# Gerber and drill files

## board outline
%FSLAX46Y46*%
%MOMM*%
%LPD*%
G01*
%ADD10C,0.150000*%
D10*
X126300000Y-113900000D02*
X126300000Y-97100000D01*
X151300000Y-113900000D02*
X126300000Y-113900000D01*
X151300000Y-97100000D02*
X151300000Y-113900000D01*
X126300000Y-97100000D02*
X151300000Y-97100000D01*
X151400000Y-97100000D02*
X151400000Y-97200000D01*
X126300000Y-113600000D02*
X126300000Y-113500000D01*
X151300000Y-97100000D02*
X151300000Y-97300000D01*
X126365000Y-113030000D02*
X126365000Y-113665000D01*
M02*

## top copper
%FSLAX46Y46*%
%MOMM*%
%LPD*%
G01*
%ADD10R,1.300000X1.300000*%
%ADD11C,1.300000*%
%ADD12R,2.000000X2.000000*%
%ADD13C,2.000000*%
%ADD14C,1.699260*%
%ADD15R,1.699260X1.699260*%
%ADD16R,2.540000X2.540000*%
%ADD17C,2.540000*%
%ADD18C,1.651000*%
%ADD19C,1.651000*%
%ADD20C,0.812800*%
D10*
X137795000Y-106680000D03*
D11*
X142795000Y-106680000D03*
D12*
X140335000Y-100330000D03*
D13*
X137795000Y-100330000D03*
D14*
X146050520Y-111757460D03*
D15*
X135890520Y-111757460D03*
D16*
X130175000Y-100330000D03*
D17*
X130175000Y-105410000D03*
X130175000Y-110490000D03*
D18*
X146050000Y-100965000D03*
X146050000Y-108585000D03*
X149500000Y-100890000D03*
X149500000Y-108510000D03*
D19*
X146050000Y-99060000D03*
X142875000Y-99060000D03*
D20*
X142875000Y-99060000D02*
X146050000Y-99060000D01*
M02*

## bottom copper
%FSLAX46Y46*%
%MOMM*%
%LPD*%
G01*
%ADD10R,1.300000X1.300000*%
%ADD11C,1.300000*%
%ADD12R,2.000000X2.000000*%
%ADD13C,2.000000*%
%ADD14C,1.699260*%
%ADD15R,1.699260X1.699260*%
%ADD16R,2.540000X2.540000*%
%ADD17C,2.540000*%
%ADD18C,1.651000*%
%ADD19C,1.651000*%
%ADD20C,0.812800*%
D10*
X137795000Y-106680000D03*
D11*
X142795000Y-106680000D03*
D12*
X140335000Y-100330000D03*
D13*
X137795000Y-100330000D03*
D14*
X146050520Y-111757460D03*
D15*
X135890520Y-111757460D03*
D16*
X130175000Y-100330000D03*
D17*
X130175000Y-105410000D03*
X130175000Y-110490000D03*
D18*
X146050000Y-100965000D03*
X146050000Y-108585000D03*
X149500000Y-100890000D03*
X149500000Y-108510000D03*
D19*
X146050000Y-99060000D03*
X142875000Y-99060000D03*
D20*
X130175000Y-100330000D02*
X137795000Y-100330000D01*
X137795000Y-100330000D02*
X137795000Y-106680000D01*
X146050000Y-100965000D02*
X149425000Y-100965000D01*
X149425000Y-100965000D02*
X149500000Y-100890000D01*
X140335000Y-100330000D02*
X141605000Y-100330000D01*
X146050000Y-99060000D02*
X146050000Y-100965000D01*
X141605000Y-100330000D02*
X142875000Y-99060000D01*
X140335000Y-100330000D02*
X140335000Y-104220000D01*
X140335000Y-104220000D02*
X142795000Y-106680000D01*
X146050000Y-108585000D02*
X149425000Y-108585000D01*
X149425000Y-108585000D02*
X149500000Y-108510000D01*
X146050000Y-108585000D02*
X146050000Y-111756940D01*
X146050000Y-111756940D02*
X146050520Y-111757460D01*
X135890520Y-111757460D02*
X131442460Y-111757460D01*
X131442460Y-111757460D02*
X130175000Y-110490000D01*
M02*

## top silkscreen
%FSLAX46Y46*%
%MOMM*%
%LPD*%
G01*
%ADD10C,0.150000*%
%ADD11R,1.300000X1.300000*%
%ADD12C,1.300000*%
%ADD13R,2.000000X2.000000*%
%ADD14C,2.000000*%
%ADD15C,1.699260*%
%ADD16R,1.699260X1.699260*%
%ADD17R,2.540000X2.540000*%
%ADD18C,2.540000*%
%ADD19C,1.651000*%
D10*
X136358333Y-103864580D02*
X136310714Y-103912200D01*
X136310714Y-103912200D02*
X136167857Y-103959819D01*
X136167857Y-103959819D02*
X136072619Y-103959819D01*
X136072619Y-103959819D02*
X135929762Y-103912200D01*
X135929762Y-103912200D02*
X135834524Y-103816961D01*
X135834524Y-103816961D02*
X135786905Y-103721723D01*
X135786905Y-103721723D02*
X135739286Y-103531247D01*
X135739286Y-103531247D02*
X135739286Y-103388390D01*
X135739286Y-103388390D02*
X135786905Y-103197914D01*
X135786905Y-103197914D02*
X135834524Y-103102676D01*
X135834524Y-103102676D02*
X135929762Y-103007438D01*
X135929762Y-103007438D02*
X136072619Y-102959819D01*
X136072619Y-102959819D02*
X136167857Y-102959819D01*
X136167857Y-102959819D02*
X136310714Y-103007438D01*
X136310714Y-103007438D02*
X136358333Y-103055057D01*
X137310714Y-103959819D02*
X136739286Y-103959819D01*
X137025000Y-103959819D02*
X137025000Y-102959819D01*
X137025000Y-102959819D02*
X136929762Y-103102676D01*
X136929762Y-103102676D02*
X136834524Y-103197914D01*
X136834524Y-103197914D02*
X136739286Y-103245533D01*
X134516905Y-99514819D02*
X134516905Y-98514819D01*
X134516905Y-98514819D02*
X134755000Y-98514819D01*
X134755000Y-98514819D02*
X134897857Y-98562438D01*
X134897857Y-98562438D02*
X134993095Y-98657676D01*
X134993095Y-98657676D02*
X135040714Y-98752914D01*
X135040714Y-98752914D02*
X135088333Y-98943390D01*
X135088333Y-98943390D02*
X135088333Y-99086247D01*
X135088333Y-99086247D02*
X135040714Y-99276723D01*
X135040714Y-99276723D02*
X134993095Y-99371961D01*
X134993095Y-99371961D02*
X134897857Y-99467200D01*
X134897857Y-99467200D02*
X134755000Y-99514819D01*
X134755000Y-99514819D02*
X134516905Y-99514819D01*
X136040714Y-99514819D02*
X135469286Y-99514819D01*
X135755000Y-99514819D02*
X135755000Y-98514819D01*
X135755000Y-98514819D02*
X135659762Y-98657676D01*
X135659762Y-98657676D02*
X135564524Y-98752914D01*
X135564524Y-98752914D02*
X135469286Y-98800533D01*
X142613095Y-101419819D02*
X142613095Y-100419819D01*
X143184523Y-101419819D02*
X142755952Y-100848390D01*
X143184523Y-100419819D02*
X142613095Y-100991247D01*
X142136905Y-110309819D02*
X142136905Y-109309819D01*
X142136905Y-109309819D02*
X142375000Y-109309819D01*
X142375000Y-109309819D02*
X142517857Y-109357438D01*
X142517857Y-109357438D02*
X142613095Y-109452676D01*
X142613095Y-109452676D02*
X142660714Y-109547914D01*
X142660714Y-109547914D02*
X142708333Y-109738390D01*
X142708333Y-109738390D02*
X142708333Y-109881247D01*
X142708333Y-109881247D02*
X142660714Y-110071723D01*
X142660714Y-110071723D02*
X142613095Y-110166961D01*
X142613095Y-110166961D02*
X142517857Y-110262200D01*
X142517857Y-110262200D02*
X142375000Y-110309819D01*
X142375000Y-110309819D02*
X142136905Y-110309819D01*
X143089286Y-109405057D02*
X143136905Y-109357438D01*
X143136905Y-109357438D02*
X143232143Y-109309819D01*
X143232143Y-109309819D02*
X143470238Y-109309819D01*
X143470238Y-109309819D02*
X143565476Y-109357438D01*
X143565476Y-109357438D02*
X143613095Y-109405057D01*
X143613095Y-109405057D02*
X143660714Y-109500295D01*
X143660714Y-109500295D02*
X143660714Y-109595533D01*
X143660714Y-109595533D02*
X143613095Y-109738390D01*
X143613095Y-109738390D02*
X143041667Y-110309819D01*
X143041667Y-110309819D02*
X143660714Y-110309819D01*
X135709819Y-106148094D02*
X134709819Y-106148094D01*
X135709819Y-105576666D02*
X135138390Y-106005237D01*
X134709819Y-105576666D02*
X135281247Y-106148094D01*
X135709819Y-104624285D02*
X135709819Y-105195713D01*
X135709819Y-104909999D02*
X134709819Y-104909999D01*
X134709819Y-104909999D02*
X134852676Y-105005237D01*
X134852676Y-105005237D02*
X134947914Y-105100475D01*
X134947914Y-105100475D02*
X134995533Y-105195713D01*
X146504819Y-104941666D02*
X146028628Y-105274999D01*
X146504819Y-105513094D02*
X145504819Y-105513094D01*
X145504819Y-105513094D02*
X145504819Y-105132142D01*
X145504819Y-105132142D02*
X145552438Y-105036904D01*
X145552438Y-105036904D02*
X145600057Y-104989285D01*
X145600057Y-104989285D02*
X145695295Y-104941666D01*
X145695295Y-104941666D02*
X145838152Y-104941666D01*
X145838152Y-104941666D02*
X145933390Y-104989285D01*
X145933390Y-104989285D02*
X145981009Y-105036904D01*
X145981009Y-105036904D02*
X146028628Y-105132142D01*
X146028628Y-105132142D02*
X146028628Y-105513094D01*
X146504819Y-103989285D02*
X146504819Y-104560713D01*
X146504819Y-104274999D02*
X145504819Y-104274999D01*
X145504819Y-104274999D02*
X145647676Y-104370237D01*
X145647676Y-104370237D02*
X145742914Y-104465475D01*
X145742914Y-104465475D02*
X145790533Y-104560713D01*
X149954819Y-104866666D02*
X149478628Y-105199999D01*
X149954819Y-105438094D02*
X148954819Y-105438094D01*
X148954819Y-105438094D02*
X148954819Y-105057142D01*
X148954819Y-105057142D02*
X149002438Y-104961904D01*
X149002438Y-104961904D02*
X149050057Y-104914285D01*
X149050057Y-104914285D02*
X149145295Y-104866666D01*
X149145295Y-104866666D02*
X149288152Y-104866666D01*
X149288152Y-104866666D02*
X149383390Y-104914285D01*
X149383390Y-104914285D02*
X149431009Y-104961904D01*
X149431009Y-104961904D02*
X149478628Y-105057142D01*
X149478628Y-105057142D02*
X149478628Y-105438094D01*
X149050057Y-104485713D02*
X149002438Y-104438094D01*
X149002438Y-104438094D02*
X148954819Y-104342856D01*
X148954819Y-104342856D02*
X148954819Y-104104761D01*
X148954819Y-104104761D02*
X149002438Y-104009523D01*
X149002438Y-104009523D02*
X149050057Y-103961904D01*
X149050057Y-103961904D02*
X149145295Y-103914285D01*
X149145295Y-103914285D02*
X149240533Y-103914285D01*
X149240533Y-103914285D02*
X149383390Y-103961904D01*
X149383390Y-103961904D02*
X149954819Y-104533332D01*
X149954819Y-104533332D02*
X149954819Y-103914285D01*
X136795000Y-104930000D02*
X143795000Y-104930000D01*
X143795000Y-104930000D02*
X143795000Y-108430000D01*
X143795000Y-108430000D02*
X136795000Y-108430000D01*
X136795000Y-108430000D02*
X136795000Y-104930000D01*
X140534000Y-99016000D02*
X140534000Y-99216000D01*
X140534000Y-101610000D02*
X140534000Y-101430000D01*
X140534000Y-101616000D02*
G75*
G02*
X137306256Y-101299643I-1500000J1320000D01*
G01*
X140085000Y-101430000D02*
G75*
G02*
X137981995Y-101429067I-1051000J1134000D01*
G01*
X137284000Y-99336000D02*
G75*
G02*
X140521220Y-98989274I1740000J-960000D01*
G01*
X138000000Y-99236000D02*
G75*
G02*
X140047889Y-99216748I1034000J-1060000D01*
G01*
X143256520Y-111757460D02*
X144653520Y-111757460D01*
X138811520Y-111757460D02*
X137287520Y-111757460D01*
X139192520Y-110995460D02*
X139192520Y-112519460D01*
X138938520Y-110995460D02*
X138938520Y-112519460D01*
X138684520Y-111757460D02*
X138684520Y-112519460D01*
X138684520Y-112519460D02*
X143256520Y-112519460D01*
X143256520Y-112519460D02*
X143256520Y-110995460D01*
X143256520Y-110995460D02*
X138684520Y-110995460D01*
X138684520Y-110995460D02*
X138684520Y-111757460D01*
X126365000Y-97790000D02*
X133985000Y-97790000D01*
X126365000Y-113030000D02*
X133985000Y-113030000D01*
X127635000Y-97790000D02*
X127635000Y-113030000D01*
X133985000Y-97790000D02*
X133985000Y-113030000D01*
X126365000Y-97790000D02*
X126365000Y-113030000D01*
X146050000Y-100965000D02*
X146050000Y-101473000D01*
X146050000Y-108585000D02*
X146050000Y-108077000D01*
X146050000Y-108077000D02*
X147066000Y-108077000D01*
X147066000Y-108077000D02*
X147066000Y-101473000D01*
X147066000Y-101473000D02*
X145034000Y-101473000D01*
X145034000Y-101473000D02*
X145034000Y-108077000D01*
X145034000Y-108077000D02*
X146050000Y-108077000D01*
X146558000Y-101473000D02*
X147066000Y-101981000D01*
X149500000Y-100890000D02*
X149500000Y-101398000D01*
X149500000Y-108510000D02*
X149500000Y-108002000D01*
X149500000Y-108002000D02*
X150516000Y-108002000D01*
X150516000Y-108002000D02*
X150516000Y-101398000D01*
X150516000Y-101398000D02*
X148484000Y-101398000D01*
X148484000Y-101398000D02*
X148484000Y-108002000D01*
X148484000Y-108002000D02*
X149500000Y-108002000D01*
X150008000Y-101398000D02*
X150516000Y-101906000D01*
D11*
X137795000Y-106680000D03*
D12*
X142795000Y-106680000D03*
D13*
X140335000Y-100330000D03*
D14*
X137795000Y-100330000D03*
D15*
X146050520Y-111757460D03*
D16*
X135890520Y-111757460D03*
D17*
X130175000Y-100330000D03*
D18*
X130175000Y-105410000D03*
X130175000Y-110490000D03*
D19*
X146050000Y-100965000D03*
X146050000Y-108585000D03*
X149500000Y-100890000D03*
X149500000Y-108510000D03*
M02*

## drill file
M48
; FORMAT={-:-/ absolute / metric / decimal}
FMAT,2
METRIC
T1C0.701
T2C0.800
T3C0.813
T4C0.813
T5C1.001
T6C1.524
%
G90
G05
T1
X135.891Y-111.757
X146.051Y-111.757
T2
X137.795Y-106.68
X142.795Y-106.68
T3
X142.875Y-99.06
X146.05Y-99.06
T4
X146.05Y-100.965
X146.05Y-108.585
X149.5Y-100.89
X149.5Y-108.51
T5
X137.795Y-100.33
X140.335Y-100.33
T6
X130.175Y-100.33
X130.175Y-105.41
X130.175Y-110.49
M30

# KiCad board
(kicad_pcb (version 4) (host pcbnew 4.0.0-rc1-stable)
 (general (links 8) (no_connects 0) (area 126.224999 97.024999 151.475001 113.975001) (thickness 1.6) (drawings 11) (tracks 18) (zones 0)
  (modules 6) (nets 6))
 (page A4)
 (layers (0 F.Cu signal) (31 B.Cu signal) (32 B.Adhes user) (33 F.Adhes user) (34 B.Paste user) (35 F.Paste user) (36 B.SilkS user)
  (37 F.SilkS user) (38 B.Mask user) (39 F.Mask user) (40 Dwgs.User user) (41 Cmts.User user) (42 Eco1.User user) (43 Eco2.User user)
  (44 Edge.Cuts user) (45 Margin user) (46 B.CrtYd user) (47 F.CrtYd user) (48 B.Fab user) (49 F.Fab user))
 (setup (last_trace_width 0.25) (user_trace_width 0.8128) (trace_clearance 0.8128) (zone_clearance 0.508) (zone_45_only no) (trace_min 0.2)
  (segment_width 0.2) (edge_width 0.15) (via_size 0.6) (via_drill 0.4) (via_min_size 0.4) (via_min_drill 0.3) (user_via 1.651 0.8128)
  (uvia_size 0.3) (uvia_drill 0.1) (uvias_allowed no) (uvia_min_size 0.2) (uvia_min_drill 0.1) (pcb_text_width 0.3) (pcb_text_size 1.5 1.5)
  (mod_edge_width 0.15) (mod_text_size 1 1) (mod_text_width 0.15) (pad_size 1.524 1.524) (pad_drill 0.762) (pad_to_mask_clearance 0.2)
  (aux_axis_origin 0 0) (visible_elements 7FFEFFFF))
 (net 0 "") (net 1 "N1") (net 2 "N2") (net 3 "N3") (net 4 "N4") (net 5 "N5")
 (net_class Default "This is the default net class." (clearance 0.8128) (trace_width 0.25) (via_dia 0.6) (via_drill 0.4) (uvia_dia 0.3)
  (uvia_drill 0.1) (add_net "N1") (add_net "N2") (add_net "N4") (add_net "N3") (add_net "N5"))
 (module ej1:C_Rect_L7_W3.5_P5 (layer F.Cu) (at 137.795 106.68)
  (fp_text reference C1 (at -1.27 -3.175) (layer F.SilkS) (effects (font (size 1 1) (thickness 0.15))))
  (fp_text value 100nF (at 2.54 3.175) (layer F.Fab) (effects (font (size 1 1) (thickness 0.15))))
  (fp_line (start -1 -1.75) (end 6 -1.75) (layer F.SilkS) (width 0.15))
  (fp_line (start 6 -1.75) (end 6 1.75) (layer F.SilkS) (width 0.15))
  (fp_line (start 6 1.75) (end -1 1.75) (layer F.SilkS) (width 0.15))
  (fp_line (start -1 1.75) (end -1 -1.75) (layer F.SilkS) (width 0.15))
  (pad 1 thru_hole rect (at 0 0) (size 1.3 1.3) (drill 0.8) (layers *.Cu *.Mask F.SilkS) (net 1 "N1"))
  (pad 2 thru_hole circle (at 5 0) (size 1.3 1.3) (drill 0.8) (layers *.Cu *.Mask F.SilkS) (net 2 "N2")))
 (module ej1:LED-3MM (layer F.Cu) (at 140.335 100.33 180)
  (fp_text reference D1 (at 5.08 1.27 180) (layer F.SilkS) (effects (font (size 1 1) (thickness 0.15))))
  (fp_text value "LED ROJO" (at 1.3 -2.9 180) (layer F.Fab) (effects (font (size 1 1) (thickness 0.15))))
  (fp_line (start -0.199 1.314) (end -0.199 1.114) (layer F.SilkS) (width 0.15))
  (fp_line (start -0.199 -1.28) (end -0.199 -1.1) (layer F.SilkS) (width 0.15))
  (fp_arc (start 1.301 0.034) (end -0.199 -1.286) (angle 108.5) (layer F.SilkS) (width 0.15))
  (fp_arc (start 1.301 0.034) (end 0.25 -1.1) (angle 85.7) (layer F.SilkS) (width 0.15))
  (fp_arc (start 1.311 0.034) (end 3.051 0.994) (angle 110) (layer F.SilkS) (width 0.15))
  (fp_arc (start 1.301 0.034) (end 2.335 1.094) (angle 87.5) (layer F.SilkS) (width 0.15))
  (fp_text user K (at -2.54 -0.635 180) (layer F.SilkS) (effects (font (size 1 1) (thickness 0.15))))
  (pad 1 thru_hole rect (at 0 0 270) (size 2 2) (drill 1.00076) (layers *.Cu *.Mask F.SilkS) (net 2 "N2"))
  (pad 2 thru_hole circle (at 2.54 0 180) (size 2 2) (drill 1.00076) (layers *.Cu *.Mask F.SilkS) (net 1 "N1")))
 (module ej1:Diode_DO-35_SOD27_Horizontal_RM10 (layer F.Cu) (at 135.89 111.76)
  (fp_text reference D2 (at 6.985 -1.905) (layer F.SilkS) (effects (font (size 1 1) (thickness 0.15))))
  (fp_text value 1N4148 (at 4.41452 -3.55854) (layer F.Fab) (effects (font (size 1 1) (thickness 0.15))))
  (fp_line (start 7.36652 -0.00254) (end 8.76352 -0.00254) (layer F.SilkS) (width 0.15))
  (fp_line (start 2.92152 -0.00254) (end 1.39752 -0.00254) (layer F.SilkS) (width 0.15))
  (fp_line (start 3.30252 -0.76454) (end 3.30252 0.75946) (layer F.SilkS) (width 0.15))
  (fp_line (start 3.04852 -0.76454) (end 3.04852 0.75946) (layer F.SilkS) (width 0.15))
  (fp_line (start 2.79452 -0.00254) (end 2.79452 0.75946) (layer F.SilkS) (width 0.15))
  (fp_line (start 2.79452 0.75946) (end 7.36652 0.75946) (layer F.SilkS) (width 0.15))
  (fp_line (start 7.36652 0.75946) (end 7.36652 -0.76454) (layer F.SilkS) (width 0.15))
  (fp_line (start 7.36652 -0.76454) (end 2.79452 -0.76454) (layer F.SilkS) (width 0.15))
  (fp_line (start 2.79452 -0.76454) (end 2.79452 -0.00254) (layer F.SilkS) (width 0.15))
  (pad 2 thru_hole circle (at 10.16052 -0.00254 180) (size 1.69926 1.69926) (drill 0.70104) (layers *.Cu *.Mask F.SilkS) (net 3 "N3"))
  (pad 1 thru_hole rect (at 0.00052 -0.00254 180) (size 1.69926 1.69926) (drill 0.70104) (layers *.Cu *.Mask F.SilkS) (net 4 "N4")))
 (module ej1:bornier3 (layer F.Cu) (at 130.175 105.41 270)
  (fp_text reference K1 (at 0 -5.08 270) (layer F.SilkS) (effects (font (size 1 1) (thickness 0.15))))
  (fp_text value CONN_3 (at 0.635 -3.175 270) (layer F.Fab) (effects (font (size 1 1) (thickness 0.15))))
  (fp_line (start -7.62 3.81) (end -7.62 -3.81) (layer F.SilkS) (width 0.15))
  (fp_line (start 7.62 3.81) (end 7.62 -3.81) (layer F.SilkS) (width 0.15))
  (fp_line (start -7.62 2.54) (end 7.62 2.54) (layer F.SilkS) (width 0.15))
  (fp_line (start -7.62 -3.81) (end 7.62 -3.81) (layer F.SilkS) (width 0.15))
  (fp_line (start -7.62 3.81) (end 7.62 3.81) (layer F.SilkS) (width 0.15))
  (pad 1 thru_hole rect (at -5.08 0 270) (size 2.54 2.54) (drill 1.524) (layers *.Cu *.Mask F.SilkS) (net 1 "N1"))
  (pad 2 thru_hole circle (at 0 0 270) (size 2.54 2.54) (drill 1.524) (layers *.Cu *.Mask F.SilkS) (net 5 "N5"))
  (pad 3 thru_hole circle (at 5.08 0 270) (size 2.54 2.54) (drill 1.524) (layers *.Cu *.Mask F.SilkS) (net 4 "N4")))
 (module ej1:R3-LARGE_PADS (layer F.Cu) (at 146.05 104.775 270)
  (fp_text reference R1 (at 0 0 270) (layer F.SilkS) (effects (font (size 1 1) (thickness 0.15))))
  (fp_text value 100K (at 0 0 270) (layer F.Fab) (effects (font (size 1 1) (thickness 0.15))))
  (fp_line (start -3.81 0) (end -3.302 0) (layer F.SilkS) (width 0.15))
  (fp_line (start 3.81 0) (end 3.302 0) (layer F.SilkS) (width 0.15))
  (fp_line (start 3.302 0) (end 3.302 -1.016) (layer F.SilkS) (width 0.15))
  (fp_line (start 3.302 -1.016) (end -3.302 -1.016) (layer F.SilkS) (width 0.15))
  (fp_line (start -3.302 -1.016) (end -3.302 1.016) (layer F.SilkS) (width 0.15))
  (fp_line (start -3.302 1.016) (end 3.302 1.016) (layer F.SilkS) (width 0.15))
  (fp_line (start 3.302 1.016) (end 3.302 0) (layer F.SilkS) (width 0.15))
  (fp_line (start -3.302 -0.508) (end -2.794 -1.016) (layer F.SilkS) (width 0.15))
  (pad 1 thru_hole circle (at -3.81 0 270) (size 1.651 1.651) (drill 0.8128) (layers *.Cu *.Mask F.SilkS) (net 2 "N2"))
  (pad 2 thru_hole circle (at 3.81 0 270) (size 1.651 1.651) (drill 0.8128) (layers *.Cu *.Mask F.SilkS) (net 3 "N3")))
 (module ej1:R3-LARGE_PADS (layer F.Cu) (at 149.5 104.7 270)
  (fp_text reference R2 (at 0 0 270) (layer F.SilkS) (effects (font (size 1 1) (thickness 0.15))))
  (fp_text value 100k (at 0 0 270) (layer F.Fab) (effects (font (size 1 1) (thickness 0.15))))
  (fp_line (start -3.81 0) (end -3.302 0) (layer F.SilkS) (width 0.15))
  (fp_line (start 3.81 0) (end 3.302 0) (layer F.SilkS) (width 0.15))
  (fp_line (start 3.302 0) (end 3.302 -1.016) (layer F.SilkS) (width 0.15))
  (fp_line (start 3.302 -1.016) (end -3.302 -1.016) (layer F.SilkS) (width 0.15))
  (fp_line (start -3.302 -1.016) (end -3.302 1.016) (layer F.SilkS) (width 0.15))
  (fp_line (start -3.302 1.016) (end 3.302 1.016) (layer F.SilkS) (width 0.15))
  (fp_line (start 3.302 1.016) (end 3.302 0) (layer F.SilkS) (width 0.15))
  (fp_line (start -3.302 -0.508) (end -2.794 -1.016) (layer F.SilkS) (width 0.15))
  (pad 1 thru_hole circle (at -3.81 0 270) (size 1.651 1.651) (drill 0.8128) (layers *.Cu *.Mask F.SilkS) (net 2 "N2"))
  (pad 2 thru_hole circle (at 3.81 0 270) (size 1.651 1.651) (drill 0.8128) (layers *.Cu *.Mask F.SilkS) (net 3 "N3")))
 (gr_line (start 126.3 113.9) (end 126.3 97.1) (angle 90) (layer Edge.Cuts) (width 0.15))
 (gr_line (start 151.3 113.9) (end 126.3 113.9) (angle 90) (layer Edge.Cuts) (width 0.15))
 (gr_line (start 151.3 97.1) (end 151.3 113.9) (angle 90) (layer Edge.Cuts) (width 0.15))
 (gr_line (start 126.3 97.1) (end 151.3 97.1) (angle 90) (layer Edge.Cuts) (width 0.15))
 (gr_line (start 151.4 97.1) (end 151.4 97.2) (angle 90) (layer Edge.Cuts) (width 0.15))
 (gr_line (start 126.3 113.6) (end 126.3 113.5) (angle 90) (layer Edge.Cuts) (width 0.15))
 (gr_line (start 151.3 97.1) (end 151.3 97.3) (angle 90) (layer Edge.Cuts) (width 0.15))
 (gr_line (start 126.365 113.03) (end 126.365 113.665) (angle 90) (layer Edge.Cuts) (width 0.15))
 (segment (start 130.175 100.33) (end 137.795 100.33) (width 0.8128) (layer B.Cu) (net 1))
 (segment (start 137.795 100.33) (end 137.795 106.68) (width 0.8128) (layer B.Cu) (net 1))
 (segment (start 146.05 100.965) (end 149.425 100.965) (width 0.8128) (layer B.Cu) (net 2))
 (segment (start 149.425 100.965) (end 149.5 100.89) (width 0.8128) (layer B.Cu) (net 2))
 (segment (start 140.335 100.33) (end 141.605 100.33) (width 0.8128) (layer B.Cu) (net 2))
 (segment (start 146.05 99.06) (end 146.05 100.965) (width 0.8128) (layer B.Cu) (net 2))
 (via (at 146.05 99.06) (size 1.651) (drill 0.8128) (layers F.Cu B.Cu) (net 2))
 (segment (start 142.875 99.06) (end 146.05 99.06) (width 0.8128) (layer F.Cu) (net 2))
 (via (at 142.875 99.06) (size 1.651) (drill 0.8128) (layers F.Cu B.Cu) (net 2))
 (segment (start 141.605 100.33) (end 142.875 99.06) (width 0.8128) (layer B.Cu) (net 2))
 (segment (start 140.335 100.33) (end 140.335 104.22) (width 0.8128) (layer B.Cu) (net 2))
 (segment (start 140.335 104.22) (end 142.795 106.68) (width 0.8128) (layer B.Cu) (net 2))
 (segment (start 146.05 108.585) (end 149.425 108.585) (width 0.8128) (layer B.Cu) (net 3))
 (segment (start 149.425 108.585) (end 149.5 108.51) (width 0.8128) (layer B.Cu) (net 3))
 (segment (start 146.05 108.585) (end 146.05 111.75694) (width 0.8128) (layer B.Cu) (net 3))
 (segment (start 146.05 111.75694) (end 146.05052 111.75746) (width 0.8128) (layer B.Cu) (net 3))
 (segment (start 135.89052 111.75746) (end 131.44246 111.75746) (width 0.8128) (layer B.Cu) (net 4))
 (segment (start 131.44246 111.75746) (end 130.175 110.49) (width 0.8128) (layer B.Cu) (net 4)))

